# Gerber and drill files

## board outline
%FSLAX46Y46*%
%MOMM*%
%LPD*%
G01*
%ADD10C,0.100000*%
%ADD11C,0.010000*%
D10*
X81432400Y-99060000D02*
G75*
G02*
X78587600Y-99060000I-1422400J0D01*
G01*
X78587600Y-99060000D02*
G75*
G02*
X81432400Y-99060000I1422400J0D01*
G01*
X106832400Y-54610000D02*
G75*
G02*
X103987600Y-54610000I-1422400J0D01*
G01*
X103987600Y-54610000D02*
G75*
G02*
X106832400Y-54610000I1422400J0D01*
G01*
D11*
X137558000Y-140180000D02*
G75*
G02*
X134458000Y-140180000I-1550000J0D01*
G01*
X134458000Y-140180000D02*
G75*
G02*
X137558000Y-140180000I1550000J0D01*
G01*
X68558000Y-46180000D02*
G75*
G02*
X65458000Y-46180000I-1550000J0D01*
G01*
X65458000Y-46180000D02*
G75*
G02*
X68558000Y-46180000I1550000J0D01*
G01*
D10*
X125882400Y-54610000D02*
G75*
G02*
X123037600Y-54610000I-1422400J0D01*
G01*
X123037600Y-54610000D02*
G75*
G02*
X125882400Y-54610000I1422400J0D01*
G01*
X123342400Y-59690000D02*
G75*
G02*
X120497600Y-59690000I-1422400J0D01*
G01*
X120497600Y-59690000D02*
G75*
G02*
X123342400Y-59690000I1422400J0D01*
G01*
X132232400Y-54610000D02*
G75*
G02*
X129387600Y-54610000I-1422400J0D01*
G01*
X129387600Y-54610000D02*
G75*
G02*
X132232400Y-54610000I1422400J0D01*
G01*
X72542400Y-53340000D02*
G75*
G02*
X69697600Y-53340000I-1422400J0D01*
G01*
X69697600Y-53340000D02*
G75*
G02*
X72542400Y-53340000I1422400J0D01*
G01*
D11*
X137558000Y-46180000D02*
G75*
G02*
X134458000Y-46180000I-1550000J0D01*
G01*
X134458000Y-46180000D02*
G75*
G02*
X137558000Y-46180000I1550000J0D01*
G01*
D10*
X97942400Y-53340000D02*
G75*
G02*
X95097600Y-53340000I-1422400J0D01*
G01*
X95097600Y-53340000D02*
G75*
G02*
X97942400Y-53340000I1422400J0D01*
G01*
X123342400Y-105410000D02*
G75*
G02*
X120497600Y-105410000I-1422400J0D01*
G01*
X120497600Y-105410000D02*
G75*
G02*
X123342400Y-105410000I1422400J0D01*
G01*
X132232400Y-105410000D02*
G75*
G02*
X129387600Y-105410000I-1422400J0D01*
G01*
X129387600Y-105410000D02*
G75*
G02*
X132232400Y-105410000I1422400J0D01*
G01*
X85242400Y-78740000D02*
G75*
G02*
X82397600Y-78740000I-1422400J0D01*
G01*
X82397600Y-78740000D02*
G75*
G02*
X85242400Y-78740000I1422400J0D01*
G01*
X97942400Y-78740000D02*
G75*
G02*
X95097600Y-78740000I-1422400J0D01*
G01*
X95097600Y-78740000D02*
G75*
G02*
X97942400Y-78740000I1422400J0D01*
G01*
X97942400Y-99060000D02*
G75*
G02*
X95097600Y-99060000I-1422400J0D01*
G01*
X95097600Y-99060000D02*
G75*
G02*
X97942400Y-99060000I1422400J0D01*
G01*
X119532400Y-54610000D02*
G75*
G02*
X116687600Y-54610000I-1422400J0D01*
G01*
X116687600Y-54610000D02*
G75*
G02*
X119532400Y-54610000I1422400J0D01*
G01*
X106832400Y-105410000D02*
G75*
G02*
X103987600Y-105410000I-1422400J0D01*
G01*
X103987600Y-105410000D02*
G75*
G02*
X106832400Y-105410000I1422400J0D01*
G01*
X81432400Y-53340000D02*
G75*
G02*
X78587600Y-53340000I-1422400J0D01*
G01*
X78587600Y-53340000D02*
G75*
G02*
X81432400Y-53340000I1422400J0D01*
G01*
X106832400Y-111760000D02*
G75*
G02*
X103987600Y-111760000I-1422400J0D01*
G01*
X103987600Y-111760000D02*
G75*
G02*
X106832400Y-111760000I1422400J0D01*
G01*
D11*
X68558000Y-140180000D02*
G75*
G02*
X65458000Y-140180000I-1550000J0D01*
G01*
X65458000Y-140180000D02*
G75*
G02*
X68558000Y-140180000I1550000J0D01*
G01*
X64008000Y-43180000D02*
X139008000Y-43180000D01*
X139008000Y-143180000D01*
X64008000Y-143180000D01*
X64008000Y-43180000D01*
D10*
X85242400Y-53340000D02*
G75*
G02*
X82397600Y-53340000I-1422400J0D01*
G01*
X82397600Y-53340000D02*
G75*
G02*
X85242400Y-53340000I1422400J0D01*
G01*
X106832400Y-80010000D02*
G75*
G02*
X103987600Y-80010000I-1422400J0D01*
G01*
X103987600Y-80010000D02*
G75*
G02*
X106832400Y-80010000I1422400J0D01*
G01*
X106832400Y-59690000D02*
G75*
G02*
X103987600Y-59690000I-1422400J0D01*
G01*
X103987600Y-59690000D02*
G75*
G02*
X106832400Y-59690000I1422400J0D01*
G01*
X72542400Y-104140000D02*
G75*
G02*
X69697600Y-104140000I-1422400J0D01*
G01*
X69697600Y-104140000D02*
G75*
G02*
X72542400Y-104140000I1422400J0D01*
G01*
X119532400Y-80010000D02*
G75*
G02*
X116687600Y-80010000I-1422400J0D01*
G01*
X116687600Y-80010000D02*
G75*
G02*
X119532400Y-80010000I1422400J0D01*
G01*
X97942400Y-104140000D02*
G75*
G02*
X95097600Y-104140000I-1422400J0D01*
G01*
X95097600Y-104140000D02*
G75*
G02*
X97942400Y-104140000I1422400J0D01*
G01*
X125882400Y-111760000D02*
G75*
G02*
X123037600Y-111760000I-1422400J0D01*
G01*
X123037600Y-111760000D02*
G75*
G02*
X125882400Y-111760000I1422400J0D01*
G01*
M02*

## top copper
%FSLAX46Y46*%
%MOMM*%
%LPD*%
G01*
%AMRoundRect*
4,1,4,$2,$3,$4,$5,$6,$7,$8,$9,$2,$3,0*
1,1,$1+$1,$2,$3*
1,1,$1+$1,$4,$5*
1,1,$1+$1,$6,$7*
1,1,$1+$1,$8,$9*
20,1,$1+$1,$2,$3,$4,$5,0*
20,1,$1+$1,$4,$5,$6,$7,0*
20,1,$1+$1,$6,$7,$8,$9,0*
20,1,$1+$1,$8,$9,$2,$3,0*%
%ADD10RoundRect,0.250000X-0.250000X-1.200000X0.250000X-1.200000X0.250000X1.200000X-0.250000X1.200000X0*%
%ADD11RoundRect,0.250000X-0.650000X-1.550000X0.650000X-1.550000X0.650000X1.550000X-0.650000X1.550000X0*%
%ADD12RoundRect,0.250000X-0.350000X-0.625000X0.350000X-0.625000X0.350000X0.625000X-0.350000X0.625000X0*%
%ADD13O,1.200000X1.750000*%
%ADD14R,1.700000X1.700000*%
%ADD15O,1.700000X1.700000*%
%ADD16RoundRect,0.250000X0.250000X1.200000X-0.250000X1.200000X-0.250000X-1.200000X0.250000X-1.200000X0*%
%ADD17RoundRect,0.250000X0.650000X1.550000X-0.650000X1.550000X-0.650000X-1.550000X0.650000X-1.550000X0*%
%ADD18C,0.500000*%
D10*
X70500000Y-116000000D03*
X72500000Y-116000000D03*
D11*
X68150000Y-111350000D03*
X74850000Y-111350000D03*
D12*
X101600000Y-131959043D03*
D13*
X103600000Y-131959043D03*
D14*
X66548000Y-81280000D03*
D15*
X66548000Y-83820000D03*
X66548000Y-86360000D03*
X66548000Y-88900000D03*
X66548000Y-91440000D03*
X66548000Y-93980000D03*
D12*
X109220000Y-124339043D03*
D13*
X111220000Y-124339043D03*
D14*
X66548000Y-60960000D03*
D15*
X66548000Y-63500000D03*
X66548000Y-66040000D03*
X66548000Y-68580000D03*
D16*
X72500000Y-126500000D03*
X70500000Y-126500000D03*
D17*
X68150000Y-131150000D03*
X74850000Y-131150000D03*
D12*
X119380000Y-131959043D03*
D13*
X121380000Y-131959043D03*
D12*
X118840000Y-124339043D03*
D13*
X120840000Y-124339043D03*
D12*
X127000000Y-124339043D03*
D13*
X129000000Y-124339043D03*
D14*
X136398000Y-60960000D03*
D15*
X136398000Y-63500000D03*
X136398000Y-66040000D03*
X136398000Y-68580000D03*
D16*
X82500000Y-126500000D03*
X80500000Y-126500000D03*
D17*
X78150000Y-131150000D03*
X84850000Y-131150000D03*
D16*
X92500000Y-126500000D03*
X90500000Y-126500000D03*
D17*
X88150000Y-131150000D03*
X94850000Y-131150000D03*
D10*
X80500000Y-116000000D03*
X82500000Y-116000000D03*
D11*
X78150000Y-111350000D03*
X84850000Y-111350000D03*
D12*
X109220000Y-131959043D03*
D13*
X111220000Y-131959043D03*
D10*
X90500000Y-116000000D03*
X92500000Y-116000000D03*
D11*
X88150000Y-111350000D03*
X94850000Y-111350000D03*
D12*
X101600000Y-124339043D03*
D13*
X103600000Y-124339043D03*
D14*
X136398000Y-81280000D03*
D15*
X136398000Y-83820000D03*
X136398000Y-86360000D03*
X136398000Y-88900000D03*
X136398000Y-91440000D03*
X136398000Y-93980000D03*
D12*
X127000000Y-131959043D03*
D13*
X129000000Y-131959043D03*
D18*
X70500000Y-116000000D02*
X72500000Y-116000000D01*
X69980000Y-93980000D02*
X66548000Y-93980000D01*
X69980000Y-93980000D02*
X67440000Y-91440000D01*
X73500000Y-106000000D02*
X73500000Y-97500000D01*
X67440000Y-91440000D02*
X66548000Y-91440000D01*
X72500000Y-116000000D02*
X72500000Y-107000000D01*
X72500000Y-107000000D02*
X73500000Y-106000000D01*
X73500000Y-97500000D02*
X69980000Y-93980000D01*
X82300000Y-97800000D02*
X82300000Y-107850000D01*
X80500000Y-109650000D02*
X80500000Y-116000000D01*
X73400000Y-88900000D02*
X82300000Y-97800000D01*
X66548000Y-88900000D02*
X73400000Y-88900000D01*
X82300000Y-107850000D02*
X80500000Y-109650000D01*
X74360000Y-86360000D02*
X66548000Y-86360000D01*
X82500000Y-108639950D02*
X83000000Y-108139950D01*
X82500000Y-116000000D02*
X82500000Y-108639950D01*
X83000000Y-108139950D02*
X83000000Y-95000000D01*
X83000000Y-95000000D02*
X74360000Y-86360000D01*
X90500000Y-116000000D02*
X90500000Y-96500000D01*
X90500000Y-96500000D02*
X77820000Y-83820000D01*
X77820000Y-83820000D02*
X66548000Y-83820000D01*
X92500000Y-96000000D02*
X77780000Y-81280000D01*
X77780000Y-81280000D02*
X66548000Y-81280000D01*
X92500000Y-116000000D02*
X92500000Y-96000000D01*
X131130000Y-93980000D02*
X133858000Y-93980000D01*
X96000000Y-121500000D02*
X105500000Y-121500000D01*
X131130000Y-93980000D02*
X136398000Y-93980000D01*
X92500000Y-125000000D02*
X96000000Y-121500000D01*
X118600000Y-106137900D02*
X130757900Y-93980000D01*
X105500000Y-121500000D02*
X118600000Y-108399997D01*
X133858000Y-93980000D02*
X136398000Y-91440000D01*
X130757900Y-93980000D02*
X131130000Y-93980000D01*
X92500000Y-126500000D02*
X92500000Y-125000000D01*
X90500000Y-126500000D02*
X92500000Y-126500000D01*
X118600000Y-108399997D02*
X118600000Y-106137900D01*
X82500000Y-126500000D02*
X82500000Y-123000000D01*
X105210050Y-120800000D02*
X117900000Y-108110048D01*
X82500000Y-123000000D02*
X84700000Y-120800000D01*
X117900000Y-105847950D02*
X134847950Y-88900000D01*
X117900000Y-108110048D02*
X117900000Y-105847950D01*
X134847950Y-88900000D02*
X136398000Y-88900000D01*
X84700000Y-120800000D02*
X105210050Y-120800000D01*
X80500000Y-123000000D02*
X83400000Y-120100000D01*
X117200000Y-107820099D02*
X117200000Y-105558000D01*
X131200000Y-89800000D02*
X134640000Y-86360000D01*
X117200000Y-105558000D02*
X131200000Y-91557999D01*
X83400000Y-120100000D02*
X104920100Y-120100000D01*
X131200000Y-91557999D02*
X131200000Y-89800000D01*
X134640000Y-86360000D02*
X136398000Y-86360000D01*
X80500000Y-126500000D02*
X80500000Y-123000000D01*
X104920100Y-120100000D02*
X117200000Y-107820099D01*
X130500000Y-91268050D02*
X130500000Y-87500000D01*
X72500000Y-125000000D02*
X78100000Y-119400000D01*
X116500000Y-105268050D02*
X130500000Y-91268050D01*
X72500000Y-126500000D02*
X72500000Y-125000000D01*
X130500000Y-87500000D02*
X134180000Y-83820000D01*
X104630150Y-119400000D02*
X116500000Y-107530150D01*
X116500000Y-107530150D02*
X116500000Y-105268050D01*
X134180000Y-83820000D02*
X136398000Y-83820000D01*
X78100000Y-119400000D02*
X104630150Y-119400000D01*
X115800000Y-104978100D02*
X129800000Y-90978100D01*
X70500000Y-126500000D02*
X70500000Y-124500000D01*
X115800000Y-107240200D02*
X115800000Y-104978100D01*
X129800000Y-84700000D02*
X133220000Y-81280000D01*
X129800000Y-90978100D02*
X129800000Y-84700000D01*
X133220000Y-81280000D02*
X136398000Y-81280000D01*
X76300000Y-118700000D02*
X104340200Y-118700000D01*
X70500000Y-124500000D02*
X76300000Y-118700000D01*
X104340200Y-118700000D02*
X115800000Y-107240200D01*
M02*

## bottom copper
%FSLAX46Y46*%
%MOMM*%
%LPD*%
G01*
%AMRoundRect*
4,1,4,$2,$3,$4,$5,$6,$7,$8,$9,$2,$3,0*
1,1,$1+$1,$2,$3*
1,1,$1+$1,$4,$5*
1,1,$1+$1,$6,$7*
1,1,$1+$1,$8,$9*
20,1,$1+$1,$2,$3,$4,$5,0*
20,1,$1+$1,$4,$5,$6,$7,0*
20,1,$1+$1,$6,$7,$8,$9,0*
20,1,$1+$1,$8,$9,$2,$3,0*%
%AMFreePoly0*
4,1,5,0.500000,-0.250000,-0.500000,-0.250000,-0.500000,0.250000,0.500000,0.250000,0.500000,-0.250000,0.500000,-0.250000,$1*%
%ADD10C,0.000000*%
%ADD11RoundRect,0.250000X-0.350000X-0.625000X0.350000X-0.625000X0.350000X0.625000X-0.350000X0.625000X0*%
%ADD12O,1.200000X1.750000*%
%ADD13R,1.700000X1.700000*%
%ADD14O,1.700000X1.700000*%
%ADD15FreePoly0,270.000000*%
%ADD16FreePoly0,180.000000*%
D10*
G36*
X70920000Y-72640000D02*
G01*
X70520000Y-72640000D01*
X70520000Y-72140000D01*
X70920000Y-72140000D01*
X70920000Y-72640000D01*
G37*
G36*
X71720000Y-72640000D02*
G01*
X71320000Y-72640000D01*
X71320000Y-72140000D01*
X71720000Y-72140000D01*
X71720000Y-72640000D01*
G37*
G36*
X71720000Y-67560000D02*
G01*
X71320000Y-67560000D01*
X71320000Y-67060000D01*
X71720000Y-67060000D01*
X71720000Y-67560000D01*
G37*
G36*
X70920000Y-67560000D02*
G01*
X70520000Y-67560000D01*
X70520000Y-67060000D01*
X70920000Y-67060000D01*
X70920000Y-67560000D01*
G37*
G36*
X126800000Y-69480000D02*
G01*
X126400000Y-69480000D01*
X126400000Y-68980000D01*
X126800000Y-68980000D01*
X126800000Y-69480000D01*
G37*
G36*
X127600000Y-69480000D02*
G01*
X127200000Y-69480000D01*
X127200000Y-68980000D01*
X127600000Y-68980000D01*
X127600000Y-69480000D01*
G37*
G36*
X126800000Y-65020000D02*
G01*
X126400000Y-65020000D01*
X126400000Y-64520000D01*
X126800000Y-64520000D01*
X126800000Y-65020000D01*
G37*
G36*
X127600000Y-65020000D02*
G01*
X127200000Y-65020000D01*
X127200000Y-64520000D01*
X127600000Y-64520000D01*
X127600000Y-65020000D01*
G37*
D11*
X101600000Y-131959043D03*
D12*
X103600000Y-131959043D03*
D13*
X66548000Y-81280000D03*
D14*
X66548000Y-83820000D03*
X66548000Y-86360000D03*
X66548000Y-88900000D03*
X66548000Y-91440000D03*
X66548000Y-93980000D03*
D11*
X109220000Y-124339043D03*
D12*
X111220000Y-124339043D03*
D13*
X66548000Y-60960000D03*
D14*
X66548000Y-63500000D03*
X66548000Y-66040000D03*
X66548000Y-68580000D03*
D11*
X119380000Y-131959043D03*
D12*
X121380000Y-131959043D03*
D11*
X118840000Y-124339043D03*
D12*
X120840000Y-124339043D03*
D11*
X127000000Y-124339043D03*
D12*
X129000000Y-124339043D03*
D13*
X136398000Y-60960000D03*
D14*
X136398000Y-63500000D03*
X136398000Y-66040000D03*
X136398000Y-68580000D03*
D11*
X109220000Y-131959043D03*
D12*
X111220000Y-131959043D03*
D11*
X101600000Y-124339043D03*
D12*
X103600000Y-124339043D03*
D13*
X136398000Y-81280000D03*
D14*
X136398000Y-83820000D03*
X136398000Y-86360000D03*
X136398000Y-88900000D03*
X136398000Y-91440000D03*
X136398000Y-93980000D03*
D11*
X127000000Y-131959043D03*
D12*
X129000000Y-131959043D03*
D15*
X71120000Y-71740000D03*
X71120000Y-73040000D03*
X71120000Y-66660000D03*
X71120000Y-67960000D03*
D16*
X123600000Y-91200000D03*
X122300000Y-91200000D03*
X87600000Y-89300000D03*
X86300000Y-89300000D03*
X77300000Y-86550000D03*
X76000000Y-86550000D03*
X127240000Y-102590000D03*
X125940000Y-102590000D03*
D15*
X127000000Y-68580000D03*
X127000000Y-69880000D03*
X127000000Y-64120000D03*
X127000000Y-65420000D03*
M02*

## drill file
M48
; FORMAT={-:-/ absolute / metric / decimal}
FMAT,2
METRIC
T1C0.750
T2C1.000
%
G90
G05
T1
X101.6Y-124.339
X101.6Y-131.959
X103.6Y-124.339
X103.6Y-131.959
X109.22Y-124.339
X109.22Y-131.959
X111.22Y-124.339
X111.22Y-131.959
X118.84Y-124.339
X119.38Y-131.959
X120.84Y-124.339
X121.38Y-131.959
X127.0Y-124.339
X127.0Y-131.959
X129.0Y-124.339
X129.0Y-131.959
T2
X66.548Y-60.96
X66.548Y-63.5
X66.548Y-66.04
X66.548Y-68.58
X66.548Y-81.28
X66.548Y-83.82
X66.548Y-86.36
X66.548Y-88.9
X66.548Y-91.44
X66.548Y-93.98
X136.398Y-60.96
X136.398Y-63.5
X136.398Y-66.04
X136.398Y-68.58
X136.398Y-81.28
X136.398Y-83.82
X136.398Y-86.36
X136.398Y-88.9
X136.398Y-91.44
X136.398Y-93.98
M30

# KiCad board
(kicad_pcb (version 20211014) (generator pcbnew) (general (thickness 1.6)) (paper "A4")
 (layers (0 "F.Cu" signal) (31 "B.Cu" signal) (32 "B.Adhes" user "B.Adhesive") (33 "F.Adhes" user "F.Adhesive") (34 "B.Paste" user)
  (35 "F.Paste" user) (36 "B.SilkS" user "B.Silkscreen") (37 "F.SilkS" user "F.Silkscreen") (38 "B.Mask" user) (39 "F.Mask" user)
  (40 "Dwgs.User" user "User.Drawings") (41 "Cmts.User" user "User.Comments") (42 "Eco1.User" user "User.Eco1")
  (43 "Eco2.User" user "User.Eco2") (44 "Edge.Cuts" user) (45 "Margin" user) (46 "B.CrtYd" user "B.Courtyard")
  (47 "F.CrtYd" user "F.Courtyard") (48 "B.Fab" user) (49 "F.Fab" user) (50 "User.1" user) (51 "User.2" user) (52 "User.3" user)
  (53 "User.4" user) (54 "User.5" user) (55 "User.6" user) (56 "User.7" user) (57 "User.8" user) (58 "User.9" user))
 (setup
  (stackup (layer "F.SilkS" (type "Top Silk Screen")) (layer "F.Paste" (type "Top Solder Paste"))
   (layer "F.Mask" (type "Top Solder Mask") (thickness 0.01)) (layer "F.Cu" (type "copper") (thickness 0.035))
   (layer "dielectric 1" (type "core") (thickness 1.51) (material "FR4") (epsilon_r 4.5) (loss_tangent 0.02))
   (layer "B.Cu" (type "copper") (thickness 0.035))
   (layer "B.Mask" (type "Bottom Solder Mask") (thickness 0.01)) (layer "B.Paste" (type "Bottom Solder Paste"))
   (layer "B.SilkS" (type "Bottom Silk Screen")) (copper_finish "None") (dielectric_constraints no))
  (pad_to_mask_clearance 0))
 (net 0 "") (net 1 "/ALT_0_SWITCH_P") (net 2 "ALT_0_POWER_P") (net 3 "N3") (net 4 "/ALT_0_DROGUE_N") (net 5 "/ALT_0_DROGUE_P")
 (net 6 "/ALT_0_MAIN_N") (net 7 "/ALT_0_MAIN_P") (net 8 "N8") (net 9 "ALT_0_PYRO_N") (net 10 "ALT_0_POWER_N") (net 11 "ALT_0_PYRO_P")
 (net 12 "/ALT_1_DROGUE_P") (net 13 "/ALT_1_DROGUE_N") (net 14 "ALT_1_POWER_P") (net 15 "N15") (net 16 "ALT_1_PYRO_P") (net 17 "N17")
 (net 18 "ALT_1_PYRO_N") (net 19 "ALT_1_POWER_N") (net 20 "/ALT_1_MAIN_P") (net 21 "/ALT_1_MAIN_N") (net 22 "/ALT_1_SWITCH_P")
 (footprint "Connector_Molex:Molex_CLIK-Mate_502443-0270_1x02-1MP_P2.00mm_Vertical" (layer "F.Cu") (at 71.5 113.5)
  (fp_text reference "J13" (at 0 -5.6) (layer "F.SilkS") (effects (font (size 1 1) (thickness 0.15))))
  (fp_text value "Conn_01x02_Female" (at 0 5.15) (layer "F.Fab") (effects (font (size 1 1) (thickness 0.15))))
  (pad "1" smd roundrect (at -1 2.5) (size 1 2.9) (layers "F.Cu" "F.Paste" "F.Mask") (roundrect_rratio 0.25) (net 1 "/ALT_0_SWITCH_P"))
  (pad "2" smd roundrect (at 1 2.5) (size 1 2.9) (layers "F.Cu" "F.Paste" "F.Mask") (roundrect_rratio 0.25) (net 1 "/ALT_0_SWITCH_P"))
  (pad "MP" smd roundrect (at -3.35 -2.15) (size 1.8 3.6) (layers "F.Cu" "F.Paste" "F.Mask") (roundrect_rratio 0.138889))
  (pad "MP" smd roundrect (at 3.35 -2.15) (size 1.8 3.6) (layers "F.Cu" "F.Paste" "F.Mask") (roundrect_rratio 0.138889)))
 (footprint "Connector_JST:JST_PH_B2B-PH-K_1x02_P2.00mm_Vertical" (layer "F.Cu") (at 101.6 131.959043)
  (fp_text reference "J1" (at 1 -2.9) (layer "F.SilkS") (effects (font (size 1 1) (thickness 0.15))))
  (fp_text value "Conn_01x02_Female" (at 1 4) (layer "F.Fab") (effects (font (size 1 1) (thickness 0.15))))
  (pad "1" thru_hole roundrect (at 0 0) (size 1.2 1.75) (drill 0.75) (layers *.Cu *.Mask) (roundrect_rratio 0.208333)
   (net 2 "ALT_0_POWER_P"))
  (pad "2" thru_hole oval (at 2 0) (size 1.2 1.75) (drill 0.75) (layers *.Cu *.Mask) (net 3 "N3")))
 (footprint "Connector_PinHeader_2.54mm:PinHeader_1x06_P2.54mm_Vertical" (layer "F.Cu") (at 66.548 81.28)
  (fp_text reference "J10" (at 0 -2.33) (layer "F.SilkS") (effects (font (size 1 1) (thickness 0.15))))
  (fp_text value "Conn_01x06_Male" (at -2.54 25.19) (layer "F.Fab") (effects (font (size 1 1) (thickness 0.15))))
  (pad "1" thru_hole rect (at 0 0) (size 1.7 1.7) (drill 1) (layers *.Cu *.Mask) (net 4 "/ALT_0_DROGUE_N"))
  (pad "2" thru_hole oval (at 0 2.54) (size 1.7 1.7) (drill 1) (layers *.Cu *.Mask) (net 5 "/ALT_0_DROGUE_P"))
  (pad "3" thru_hole oval (at 0 5.08) (size 1.7 1.7) (drill 1) (layers *.Cu *.Mask) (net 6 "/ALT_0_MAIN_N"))
  (pad "4" thru_hole oval (at 0 7.62) (size 1.7 1.7) (drill 1) (layers *.Cu *.Mask) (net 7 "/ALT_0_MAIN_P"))
  (pad "5" thru_hole oval (at 0 10.16) (size 1.7 1.7) (drill 1) (layers *.Cu *.Mask) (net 1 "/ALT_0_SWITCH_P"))
  (pad "6" thru_hole oval (at 0 12.7) (size 1.7 1.7) (drill 1) (layers *.Cu *.Mask) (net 1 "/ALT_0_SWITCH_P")))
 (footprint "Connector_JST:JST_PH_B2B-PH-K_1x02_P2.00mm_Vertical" (layer "F.Cu") (at 109.22 124.339043)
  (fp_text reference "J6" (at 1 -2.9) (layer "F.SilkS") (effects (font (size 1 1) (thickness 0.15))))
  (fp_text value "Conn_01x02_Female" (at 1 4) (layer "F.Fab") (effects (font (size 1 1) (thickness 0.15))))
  (pad "1" thru_hole roundrect (at 0 0) (size 1.2 1.75) (drill 0.75) (layers *.Cu *.Mask) (roundrect_rratio 0.208333) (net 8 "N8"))
  (pad "2" thru_hole oval (at 2 0) (size 1.2 1.75) (drill 0.75) (layers *.Cu *.Mask) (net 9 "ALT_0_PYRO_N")))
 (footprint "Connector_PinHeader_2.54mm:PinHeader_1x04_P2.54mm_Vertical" (layer "F.Cu") (at 66.548 60.96)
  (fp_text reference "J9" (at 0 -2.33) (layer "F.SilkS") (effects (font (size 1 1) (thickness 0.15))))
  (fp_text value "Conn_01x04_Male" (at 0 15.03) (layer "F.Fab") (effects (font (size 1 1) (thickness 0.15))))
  (pad "1" thru_hole rect (at 0 0) (size 1.7 1.7) (drill 1) (layers *.Cu *.Mask) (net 2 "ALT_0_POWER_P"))
  (pad "2" thru_hole oval (at 0 2.54) (size 1.7 1.7) (drill 1) (layers *.Cu *.Mask) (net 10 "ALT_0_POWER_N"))
  (pad "3" thru_hole oval (at 0 5.08) (size 1.7 1.7) (drill 1) (layers *.Cu *.Mask) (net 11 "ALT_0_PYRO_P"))
  (pad "4" thru_hole oval (at 0 7.62) (size 1.7 1.7) (drill 1) (layers *.Cu *.Mask) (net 9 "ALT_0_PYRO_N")))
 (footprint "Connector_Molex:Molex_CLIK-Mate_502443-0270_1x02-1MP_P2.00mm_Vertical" (layer "F.Cu") (at 71.5 129 180)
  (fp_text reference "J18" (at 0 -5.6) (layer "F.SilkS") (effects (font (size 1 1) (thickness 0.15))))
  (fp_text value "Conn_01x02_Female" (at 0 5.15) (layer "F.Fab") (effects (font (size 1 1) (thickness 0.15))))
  (pad "1" smd roundrect (at -1 2.5 180) (size 1 2.9) (layers "F.Cu" "F.Paste" "F.Mask") (roundrect_rratio 0.25) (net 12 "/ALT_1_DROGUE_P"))
  (pad "2" smd roundrect (at 1 2.5 180) (size 1 2.9) (layers "F.Cu" "F.Paste" "F.Mask") (roundrect_rratio 0.25) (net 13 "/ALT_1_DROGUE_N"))
  (pad "MP" smd roundrect (at 3.35 -2.15 180) (size 1.8 3.6) (layers "F.Cu" "F.Paste" "F.Mask") (roundrect_rratio 0.138889))
  (pad "MP" smd roundrect (at -3.35 -2.15 180) (size 1.8 3.6) (layers "F.Cu" "F.Paste" "F.Mask") (roundrect_rratio 0.138889)))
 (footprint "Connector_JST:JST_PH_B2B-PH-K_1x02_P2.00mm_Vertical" (layer "F.Cu") (at 119.38 131.959043)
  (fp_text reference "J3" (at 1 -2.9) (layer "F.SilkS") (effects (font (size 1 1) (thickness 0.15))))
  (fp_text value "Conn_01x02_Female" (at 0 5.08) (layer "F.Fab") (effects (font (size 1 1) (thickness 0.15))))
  (pad "1" thru_hole roundrect (at 0 0) (size 1.2 1.75) (drill 0.75) (layers *.Cu *.Mask) (roundrect_rratio 0.208333)
   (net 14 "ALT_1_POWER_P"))
  (pad "2" thru_hole oval (at 2 0) (size 1.2 1.75) (drill 0.75) (layers *.Cu *.Mask) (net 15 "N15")))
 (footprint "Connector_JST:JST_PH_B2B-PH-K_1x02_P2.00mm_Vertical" (layer "F.Cu") (at 118.84 124.339043)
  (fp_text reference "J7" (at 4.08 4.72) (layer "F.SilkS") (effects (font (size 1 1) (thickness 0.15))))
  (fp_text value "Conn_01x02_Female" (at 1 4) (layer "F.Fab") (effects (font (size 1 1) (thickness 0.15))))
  (pad "1" thru_hole roundrect (at 0 0) (size 1.2 1.75) (drill 0.75) (layers *.Cu *.Mask) (roundrect_rratio 0.208333)
   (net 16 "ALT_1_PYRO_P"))
  (pad "2" thru_hole oval (at 2 0) (size 1.2 1.75) (drill 0.75) (layers *.Cu *.Mask) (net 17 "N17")))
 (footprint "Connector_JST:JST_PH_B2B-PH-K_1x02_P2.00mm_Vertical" (layer "F.Cu") (at 127 124.339043)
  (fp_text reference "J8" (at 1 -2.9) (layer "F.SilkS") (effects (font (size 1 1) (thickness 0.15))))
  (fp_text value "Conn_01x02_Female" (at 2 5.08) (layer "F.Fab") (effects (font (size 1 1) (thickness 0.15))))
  (pad "1" thru_hole roundrect (at 0 0) (size 1.2 1.75) (drill 0.75) (layers *.Cu *.Mask) (roundrect_rratio 0.208333) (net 17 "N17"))
  (pad "2" thru_hole oval (at 2 0) (size 1.2 1.75) (drill 0.75) (layers *.Cu *.Mask) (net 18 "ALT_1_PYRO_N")))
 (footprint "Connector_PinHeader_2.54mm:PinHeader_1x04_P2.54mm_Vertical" (layer "F.Cu") (at 136.398 60.96)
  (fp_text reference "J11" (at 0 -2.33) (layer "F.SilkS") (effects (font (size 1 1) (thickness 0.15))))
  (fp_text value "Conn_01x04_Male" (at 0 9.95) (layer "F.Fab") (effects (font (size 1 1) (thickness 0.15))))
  (pad "1" thru_hole rect (at 0 0) (size 1.7 1.7) (drill 1) (layers *.Cu *.Mask) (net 14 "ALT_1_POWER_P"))
  (pad "2" thru_hole oval (at 0 2.54) (size 1.7 1.7) (drill 1) (layers *.Cu *.Mask) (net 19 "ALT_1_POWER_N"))
  (pad "3" thru_hole oval (at 0 5.08) (size 1.7 1.7) (drill 1) (layers *.Cu *.Mask) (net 16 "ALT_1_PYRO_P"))
  (pad "4" thru_hole oval (at 0 7.62) (size 1.7 1.7) (drill 1) (layers *.Cu *.Mask) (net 18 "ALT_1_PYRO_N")))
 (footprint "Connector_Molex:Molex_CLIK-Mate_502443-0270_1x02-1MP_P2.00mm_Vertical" (layer "F.Cu") (at 81.5 129 180)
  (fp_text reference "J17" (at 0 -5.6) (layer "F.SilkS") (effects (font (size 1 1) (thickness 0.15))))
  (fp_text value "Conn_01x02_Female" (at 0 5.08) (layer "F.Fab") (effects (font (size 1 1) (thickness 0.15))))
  (pad "1" smd roundrect (at -1 2.5 180) (size 1 2.9) (layers "F.Cu" "F.Paste" "F.Mask") (roundrect_rratio 0.25) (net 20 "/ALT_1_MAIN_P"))
  (pad "2" smd roundrect (at 1 2.5 180) (size 1 2.9) (layers "F.Cu" "F.Paste" "F.Mask") (roundrect_rratio 0.25) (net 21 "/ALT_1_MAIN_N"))
  (pad "MP" smd roundrect (at 3.35 -2.15 180) (size 1.8 3.6) (layers "F.Cu" "F.Paste" "F.Mask") (roundrect_rratio 0.138889))
  (pad "MP" smd roundrect (at -3.35 -2.15 180) (size 1.8 3.6) (layers "F.Cu" "F.Paste" "F.Mask") (roundrect_rratio 0.138889)))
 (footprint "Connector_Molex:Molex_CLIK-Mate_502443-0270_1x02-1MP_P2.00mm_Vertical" (layer "F.Cu") (at 91.5 129 180)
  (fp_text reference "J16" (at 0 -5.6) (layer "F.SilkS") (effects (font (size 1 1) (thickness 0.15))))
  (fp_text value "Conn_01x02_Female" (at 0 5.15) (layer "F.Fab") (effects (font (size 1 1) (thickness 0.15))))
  (pad "1" smd roundrect (at -1 2.5 180) (size 1 2.9) (layers "F.Cu" "F.Paste" "F.Mask") (roundrect_rratio 0.25) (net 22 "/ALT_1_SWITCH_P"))
  (pad "2" smd roundrect (at 1 2.5 180) (size 1 2.9) (layers "F.Cu" "F.Paste" "F.Mask") (roundrect_rratio 0.25) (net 22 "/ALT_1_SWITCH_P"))
  (pad "MP" smd roundrect (at 3.35 -2.15 180) (size 1.8 3.6) (layers "F.Cu" "F.Paste" "F.Mask") (roundrect_rratio 0.138889))
  (pad "MP" smd roundrect (at -3.35 -2.15 180) (size 1.8 3.6) (layers "F.Cu" "F.Paste" "F.Mask") (roundrect_rratio 0.138889)))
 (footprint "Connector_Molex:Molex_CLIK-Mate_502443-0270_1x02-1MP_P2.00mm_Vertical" (layer "F.Cu") (at 81.5 113.5)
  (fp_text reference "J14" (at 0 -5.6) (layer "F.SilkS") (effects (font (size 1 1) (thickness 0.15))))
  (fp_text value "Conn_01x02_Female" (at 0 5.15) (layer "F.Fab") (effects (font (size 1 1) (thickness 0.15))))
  (pad "1" smd roundrect (at -1 2.5) (size 1 2.9) (layers "F.Cu" "F.Paste" "F.Mask") (roundrect_rratio 0.25) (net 7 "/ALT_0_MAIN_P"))
  (pad "2" smd roundrect (at 1 2.5) (size 1 2.9) (layers "F.Cu" "F.Paste" "F.Mask") (roundrect_rratio 0.25) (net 6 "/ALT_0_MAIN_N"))
  (pad "MP" smd roundrect (at -3.35 -2.15) (size 1.8 3.6) (layers "F.Cu" "F.Paste" "F.Mask") (roundrect_rratio 0.138889))
  (pad "MP" smd roundrect (at 3.35 -2.15) (size 1.8 3.6) (layers "F.Cu" "F.Paste" "F.Mask") (roundrect_rratio 0.138889)))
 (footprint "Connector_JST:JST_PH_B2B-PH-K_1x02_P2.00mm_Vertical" (layer "F.Cu") (at 109.22 131.959043)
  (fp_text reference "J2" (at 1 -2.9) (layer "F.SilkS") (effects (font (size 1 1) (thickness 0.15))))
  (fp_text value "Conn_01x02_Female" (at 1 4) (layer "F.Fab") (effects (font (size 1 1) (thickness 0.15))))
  (pad "1" thru_hole roundrect (at 0 0) (size 1.2 1.75) (drill 0.75) (layers *.Cu *.Mask) (roundrect_rratio 0.208333) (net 3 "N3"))
  (pad "2" thru_hole oval (at 2 0) (size 1.2 1.75) (drill 0.75) (layers *.Cu *.Mask) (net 10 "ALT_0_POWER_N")))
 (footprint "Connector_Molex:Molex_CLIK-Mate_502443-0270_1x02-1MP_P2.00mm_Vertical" (layer "F.Cu") (at 91.5 113.5)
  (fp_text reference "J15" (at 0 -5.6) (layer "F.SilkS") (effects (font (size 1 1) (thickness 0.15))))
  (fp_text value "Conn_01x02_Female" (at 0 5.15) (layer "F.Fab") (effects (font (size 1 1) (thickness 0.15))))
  (pad "1" smd roundrect (at -1 2.5) (size 1 2.9) (layers "F.Cu" "F.Paste" "F.Mask") (roundrect_rratio 0.25) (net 5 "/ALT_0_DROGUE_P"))
  (pad "2" smd roundrect (at 1 2.5) (size 1 2.9) (layers "F.Cu" "F.Paste" "F.Mask") (roundrect_rratio 0.25) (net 4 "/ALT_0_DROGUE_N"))
  (pad "MP" smd roundrect (at -3.35 -2.15) (size 1.8 3.6) (layers "F.Cu" "F.Paste" "F.Mask") (roundrect_rratio 0.138889))
  (pad "MP" smd roundrect (at 3.35 -2.15) (size 1.8 3.6) (layers "F.Cu" "F.Paste" "F.Mask") (roundrect_rratio 0.138889)))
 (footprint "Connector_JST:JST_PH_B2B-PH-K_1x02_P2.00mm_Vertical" (layer "F.Cu") (at 101.6 124.339043)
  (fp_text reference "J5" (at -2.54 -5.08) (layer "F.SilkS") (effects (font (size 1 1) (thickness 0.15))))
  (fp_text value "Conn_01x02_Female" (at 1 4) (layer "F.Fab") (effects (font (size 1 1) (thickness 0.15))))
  (pad "1" thru_hole roundrect (at 0 0) (size 1.2 1.75) (drill 0.75) (layers *.Cu *.Mask) (roundrect_rratio 0.208333)
   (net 11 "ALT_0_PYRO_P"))
  (pad "2" thru_hole oval (at 2 0) (size 1.2 1.75) (drill 0.75) (layers *.Cu *.Mask) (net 8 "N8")))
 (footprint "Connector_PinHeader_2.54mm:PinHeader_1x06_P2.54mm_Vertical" (layer "F.Cu") (at 136.398 81.28)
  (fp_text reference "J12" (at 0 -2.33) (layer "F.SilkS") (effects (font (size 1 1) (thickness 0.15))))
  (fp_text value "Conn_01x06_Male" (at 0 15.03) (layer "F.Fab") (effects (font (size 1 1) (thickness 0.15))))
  (pad "1" thru_hole rect (at 0 0) (size 1.7 1.7) (drill 1) (layers *.Cu *.Mask) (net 13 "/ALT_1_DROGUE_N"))
  (pad "2" thru_hole oval (at 0 2.54) (size 1.7 1.7) (drill 1) (layers *.Cu *.Mask) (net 12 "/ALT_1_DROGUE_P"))
  (pad "3" thru_hole oval (at 0 5.08) (size 1.7 1.7) (drill 1) (layers *.Cu *.Mask) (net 21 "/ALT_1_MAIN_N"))
  (pad "4" thru_hole oval (at 0 7.62) (size 1.7 1.7) (drill 1) (layers *.Cu *.Mask) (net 20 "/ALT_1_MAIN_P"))
  (pad "5" thru_hole oval (at 0 10.16) (size 1.7 1.7) (drill 1) (layers *.Cu *.Mask) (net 22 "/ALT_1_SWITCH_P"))
  (pad "6" thru_hole oval (at 0 12.7) (size 1.7 1.7) (drill 1) (layers *.Cu *.Mask) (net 22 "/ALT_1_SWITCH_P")))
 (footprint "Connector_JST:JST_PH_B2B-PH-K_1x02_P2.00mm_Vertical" (layer "F.Cu") (at 127 131.959043)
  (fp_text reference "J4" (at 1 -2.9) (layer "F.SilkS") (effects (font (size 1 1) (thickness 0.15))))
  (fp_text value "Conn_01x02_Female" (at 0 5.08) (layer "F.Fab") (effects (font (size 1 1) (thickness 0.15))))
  (pad "1" thru_hole roundrect (at 0 0) (size 1.2 1.75) (drill 0.75) (layers *.Cu *.Mask) (roundrect_rratio 0.208333) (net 15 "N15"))
  (pad "2" thru_hole oval (at 2 0) (size 1.2 1.75) (drill 0.75) (layers *.Cu *.Mask) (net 19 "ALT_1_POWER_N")))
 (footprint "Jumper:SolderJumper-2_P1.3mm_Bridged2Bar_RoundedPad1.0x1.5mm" (layer "B.Cu") (at 71.12 72.39 -90)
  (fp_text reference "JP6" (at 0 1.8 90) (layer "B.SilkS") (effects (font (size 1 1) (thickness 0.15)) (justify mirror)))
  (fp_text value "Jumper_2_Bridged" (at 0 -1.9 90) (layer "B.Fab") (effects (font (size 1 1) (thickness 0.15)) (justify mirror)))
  (fp_poly (pts (xy -0.25 0.6) (xy 0.25 0.6) (xy 0.25 0.2) (xy -0.25 0.2)) (layer "B.Cu") (width 0) (fill solid))
  (fp_poly (pts (xy -0.25 -0.2) (xy 0.25 -0.2) (xy 0.25 -0.6) (xy -0.25 -0.6)) (layer "B.Cu") (width 0) (fill solid))
  (pad "1" smd custom (at -0.65 0 270) (size 1 0.5) (layers "B.Cu" "B.Mask") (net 10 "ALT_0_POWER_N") (zone_connect 2)
   (options (clearance outline) (anchor rect)) (primitives))
  (pad "2" smd custom (at 0.65 0 270) (size 1 0.5) (layers "B.Cu" "B.Mask") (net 9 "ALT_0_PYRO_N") (zone_connect 2)
   (options (clearance outline) (anchor rect)) (primitives)))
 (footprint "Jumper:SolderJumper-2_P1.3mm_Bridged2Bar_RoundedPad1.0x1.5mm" (layer "B.Cu") (at 71.12 67.31 -90)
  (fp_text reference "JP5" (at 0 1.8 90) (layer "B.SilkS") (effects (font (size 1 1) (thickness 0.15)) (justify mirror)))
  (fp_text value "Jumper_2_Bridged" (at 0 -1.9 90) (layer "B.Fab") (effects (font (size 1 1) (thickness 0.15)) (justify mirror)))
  (fp_poly (pts (xy -0.25 -0.2) (xy 0.25 -0.2) (xy 0.25 -0.6) (xy -0.25 -0.6)) (layer "B.Cu") (width 0) (fill solid))
  (fp_poly (pts (xy -0.25 0.6) (xy 0.25 0.6) (xy 0.25 0.2) (xy -0.25 0.2)) (layer "B.Cu") (width 0) (fill solid))
  (pad "1" smd custom (at -0.65 0 270) (size 1 0.5) (layers "B.Cu" "B.Mask") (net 2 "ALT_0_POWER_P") (zone_connect 2)
   (options (clearance outline) (anchor rect)) (primitives))
  (pad "2" smd custom (at 0.65 0 270) (size 1 0.5) (layers "B.Cu" "B.Mask") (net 11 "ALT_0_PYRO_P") (zone_connect 2)
   (options (clearance outline) (anchor rect)) (primitives)))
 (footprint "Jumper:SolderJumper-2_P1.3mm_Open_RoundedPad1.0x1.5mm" (layer "B.Cu") (at 122.95 91.2 180)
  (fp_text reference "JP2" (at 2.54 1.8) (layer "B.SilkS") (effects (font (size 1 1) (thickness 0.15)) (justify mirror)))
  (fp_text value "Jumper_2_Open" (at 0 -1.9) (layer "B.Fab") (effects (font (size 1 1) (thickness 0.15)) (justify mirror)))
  (pad "1" smd custom (at -0.65 0 180) (size 1 0.5) (layers "B.Cu" "B.Mask") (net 19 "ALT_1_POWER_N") (zone_connect 2)
   (options (clearance outline) (anchor rect)) (primitives))
  (pad "2" smd custom (at 0.65 0 180) (size 1 0.5) (layers "B.Cu" "B.Mask") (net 15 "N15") (zone_connect 2)
   (options (clearance outline) (anchor rect)) (primitives)))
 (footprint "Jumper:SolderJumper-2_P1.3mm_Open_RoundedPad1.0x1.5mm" (layer "B.Cu") (at 86.95 89.3 180)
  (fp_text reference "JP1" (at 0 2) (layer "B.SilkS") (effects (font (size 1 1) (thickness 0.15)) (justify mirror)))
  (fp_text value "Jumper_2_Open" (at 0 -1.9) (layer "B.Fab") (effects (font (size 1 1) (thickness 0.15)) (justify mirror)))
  (pad "1" smd custom (at -0.65 0 180) (size 1 0.5) (layers "B.Cu" "B.Mask") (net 10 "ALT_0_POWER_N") (zone_connect 2)
   (options (clearance outline) (anchor rect)) (primitives))
  (pad "2" smd custom (at 0.65 0 180) (size 1 0.5) (layers "B.Cu" "B.Mask") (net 3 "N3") (zone_connect 2)
   (options (clearance outline) (anchor rect)) (primitives)))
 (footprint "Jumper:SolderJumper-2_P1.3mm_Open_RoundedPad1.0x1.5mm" (layer "B.Cu") (at 76.65 86.55 180)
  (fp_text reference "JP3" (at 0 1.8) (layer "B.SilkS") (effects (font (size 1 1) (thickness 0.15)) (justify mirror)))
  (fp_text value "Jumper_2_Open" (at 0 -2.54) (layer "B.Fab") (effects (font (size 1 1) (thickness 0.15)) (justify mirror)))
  (pad "1" smd custom (at -0.65 0 180) (size 1 0.5) (layers "B.Cu" "B.Mask") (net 9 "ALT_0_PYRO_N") (zone_connect 2)
   (options (clearance outline) (anchor rect)) (primitives))
  (pad "2" smd custom (at 0.65 0 180) (size 1 0.5) (layers "B.Cu" "B.Mask") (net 8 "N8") (zone_connect 2)
   (options (clearance outline) (anchor rect)) (primitives)))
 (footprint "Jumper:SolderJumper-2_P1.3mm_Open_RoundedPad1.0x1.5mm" (layer "B.Cu") (at 126.59 102.59 180)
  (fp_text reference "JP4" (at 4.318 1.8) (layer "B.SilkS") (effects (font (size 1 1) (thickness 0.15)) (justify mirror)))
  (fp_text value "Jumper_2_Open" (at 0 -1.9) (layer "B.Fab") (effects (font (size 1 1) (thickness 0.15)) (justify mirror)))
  (pad "1" smd custom (at -0.65 0 180) (size 1 0.5) (layers "B.Cu" "B.Mask") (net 18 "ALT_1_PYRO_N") (zone_connect 2)
   (options (clearance outline) (anchor rect)) (primitives))
  (pad "2" smd custom (at 0.65 0 180) (size 1 0.5) (layers "B.Cu" "B.Mask") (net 17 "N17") (zone_connect 2)
   (options (clearance outline) (anchor rect)) (primitives)))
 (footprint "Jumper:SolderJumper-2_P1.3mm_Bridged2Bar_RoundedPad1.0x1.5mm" (layer "B.Cu") (at 127 69.23 -90)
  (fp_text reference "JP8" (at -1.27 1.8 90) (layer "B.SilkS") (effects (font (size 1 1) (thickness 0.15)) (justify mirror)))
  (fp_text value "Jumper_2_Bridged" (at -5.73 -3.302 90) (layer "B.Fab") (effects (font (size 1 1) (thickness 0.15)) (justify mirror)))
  (fp_poly (pts (xy -0.25 0.6) (xy 0.25 0.6) (xy 0.25 0.2) (xy -0.25 0.2)) (layer "B.Cu") (width 0) (fill solid))
  (fp_poly (pts (xy -0.25 -0.2) (xy 0.25 -0.2) (xy 0.25 -0.6) (xy -0.25 -0.6)) (layer "B.Cu") (width 0) (fill solid))
  (pad "1" smd custom (at -0.65 0 270) (size 1 0.5) (layers "B.Cu" "B.Mask") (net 19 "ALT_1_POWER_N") (zone_connect 2)
   (options (clearance outline) (anchor rect)) (primitives))
  (pad "2" smd custom (at 0.65 0 270) (size 1 0.5) (layers "B.Cu" "B.Mask") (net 18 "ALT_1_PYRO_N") (zone_connect 2)
   (options (clearance outline) (anchor rect)) (primitives)))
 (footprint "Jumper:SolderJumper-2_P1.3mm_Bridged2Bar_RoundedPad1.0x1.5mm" (layer "B.Cu") (at 127 64.77 -90)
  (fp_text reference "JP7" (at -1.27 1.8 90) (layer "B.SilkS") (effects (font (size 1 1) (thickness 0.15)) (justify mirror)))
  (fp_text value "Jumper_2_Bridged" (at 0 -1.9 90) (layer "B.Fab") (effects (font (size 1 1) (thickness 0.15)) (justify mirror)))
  (fp_poly (pts (xy -0.25 0.6) (xy 0.25 0.6) (xy 0.25 0.2) (xy -0.25 0.2)) (layer "B.Cu") (width 0) (fill solid))
  (fp_poly (pts (xy -0.25 -0.2) (xy 0.25 -0.2) (xy 0.25 -0.6) (xy -0.25 -0.6)) (layer "B.Cu") (width 0) (fill solid))
  (pad "1" smd custom (at -0.65 0 270) (size 1 0.5) (layers "B.Cu" "B.Mask") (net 14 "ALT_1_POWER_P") (zone_connect 2)
   (options (clearance outline) (anchor rect)) (primitives))
  (pad "2" smd custom (at 0.65 0 270) (size 1 0.5) (layers "B.Cu" "B.Mask") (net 16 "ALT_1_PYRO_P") (zone_connect 2)
   (options (clearance outline) (anchor rect)) (primitives)))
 (gr_circle (center 80.01 99.06) (end 81.4324 99.06) (layer "Edge.Cuts") (width 0.1) (fill none))
 (gr_circle (center 105.41 54.61) (end 106.8324 54.61) (layer "Edge.Cuts") (width 0.1) (fill none))
 (gr_circle (center 136.008 140.18) (end 137.558 140.18) (layer "Edge.Cuts") (width 0.01) (fill none))
 (gr_circle (center 67.008 46.18) (end 68.558 46.18) (layer "Edge.Cuts") (width 0.01) (fill none))
 (gr_circle (center 124.46 54.61) (end 125.8824 54.61) (layer "Edge.Cuts") (width 0.1) (fill none))
 (gr_circle (center 121.92 59.69) (end 123.3424 59.69) (layer "Edge.Cuts") (width 0.1) (fill none))
 (gr_circle (center 130.81 54.61) (end 132.2324 54.61) (layer "Edge.Cuts") (width 0.1) (fill none))
 (gr_circle (center 71.12 53.34) (end 72.5424 53.34) (layer "Edge.Cuts") (width 0.1) (fill none))
 (gr_circle (center 136.008 46.18) (end 137.558 46.18) (layer "Edge.Cuts") (width 0.01) (fill none))
 (gr_circle (center 96.52 53.34) (end 97.9424 53.34) (layer "Edge.Cuts") (width 0.1) (fill none))
 (gr_circle (center 121.92 105.41) (end 123.3424 105.41) (layer "Edge.Cuts") (width 0.1) (fill none))
 (gr_circle (center 130.81 105.41) (end 132.2324 105.41) (layer "Edge.Cuts") (width 0.1) (fill none))
 (gr_circle (center 83.82 78.74) (end 85.2424 78.74) (layer "Edge.Cuts") (width 0.1) (fill none))
 (gr_circle (center 96.52 78.74) (end 97.9424 78.74) (layer "Edge.Cuts") (width 0.1) (fill none))
 (gr_circle (center 96.52 99.06) (end 97.9424 99.06) (layer "Edge.Cuts") (width 0.1) (fill none))
 (gr_circle (center 118.11 54.61) (end 119.5324 54.61) (layer "Edge.Cuts") (width 0.1) (fill none))
 (gr_circle (center 105.41 105.41) (end 106.8324 105.41) (layer "Edge.Cuts") (width 0.1) (fill none))
 (gr_circle (center 80.01 53.34) (end 81.4324 53.34) (layer "Edge.Cuts") (width 0.1) (fill none))
 (gr_circle (center 105.41 111.76) (end 106.8324 111.76) (layer "Edge.Cuts") (width 0.1) (fill none))
 (gr_circle (center 67.008 140.18) (end 68.558 140.18) (layer "Edge.Cuts") (width 0.01) (fill none))
 (gr_rect (start 64.008 43.18) (end 139.008 143.18) (layer "Edge.Cuts") (width 0.01) (fill none))
 (gr_circle (center 83.82 53.34) (end 85.2424 53.34) (layer "Edge.Cuts") (width 0.1) (fill none))
 (gr_circle (center 105.41 80.01) (end 106.8324 80.01) (layer "Edge.Cuts") (width 0.1) (fill none))
 (gr_circle (center 105.41 59.69) (end 106.8324 59.69) (layer "Edge.Cuts") (width 0.1) (fill none))
 (gr_circle (center 71.12 104.14) (end 72.5424 104.14) (layer "Edge.Cuts") (width 0.1) (fill none))
 (gr_circle (center 118.11 80.01) (end 119.5324 80.01) (layer "Edge.Cuts") (width 0.1) (fill none))
 (gr_circle (center 96.52 104.14) (end 97.9424 104.14) (layer "Edge.Cuts") (width 0.1) (fill none))
 (gr_circle (center 124.46 111.76) (end 125.8824 111.76) (layer "Edge.Cuts") (width 0.1) (fill none))
 (segment (start 70.5 116) (end 72.5 116) (width 0.5) (layer "F.Cu") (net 1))
 (segment (start 69.98 93.98) (end 66.548 93.98) (width 0.5) (layer "F.Cu") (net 1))
 (segment (start 69.98 93.98) (end 67.44 91.44) (width 0.5) (layer "F.Cu") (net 1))
 (segment (start 73.5 106) (end 73.5 97.5) (width 0.5) (layer "F.Cu") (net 1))
 (segment (start 67.44 91.44) (end 66.548 91.44) (width 0.5) (layer "F.Cu") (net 1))
 (segment (start 72.5 116) (end 72.5 107) (width 0.5) (layer "F.Cu") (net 1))
 (segment (start 72.5 107) (end 73.5 106) (width 0.5) (layer "F.Cu") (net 1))
 (segment (start 73.5 97.5) (end 69.98 93.98) (width 0.5) (layer "F.Cu") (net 1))
 (segment (start 82.3 97.8) (end 82.3 107.85) (width 0.5) (layer "F.Cu") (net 7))
 (segment (start 80.5 109.65) (end 80.5 116) (width 0.5) (layer "F.Cu") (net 7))
 (segment (start 73.4 88.9) (end 82.3 97.8) (width 0.5) (layer "F.Cu") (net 7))
 (segment (start 66.548 88.9) (end 73.4 88.9) (width 0.5) (layer "F.Cu") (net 7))
 (segment (start 82.3 107.85) (end 80.5 109.65) (width 0.5) (layer "F.Cu") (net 7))
 (segment (start 74.36 86.36) (end 66.548 86.36) (width 0.5) (layer "F.Cu") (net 6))
 (segment (start 82.5 108.63995) (end 83 108.13995) (width 0.5) (layer "F.Cu") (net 6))
 (segment (start 82.5 116) (end 82.5 108.63995) (width 0.5) (layer "F.Cu") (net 6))
 (segment (start 83 108.13995) (end 83 95) (width 0.5) (layer "F.Cu") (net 6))
 (segment (start 83 95) (end 74.36 86.36) (width 0.5) (layer "F.Cu") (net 6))
 (segment (start 90.5 116) (end 90.5 96.5) (width 0.5) (layer "F.Cu") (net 5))
 (segment (start 90.5 96.5) (end 77.82 83.82) (width 0.5) (layer "F.Cu") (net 5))
 (segment (start 77.82 83.82) (end 66.548 83.82) (width 0.5) (layer "F.Cu") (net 5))
 (segment (start 92.5 96) (end 77.78 81.28) (width 0.5) (layer "F.Cu") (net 4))
 (segment (start 77.78 81.28) (end 66.548 81.28) (width 0.5) (layer "F.Cu") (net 4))
 (segment (start 92.5 116) (end 92.5 96) (width 0.5) (layer "F.Cu") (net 4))
 (segment (start 131.13 93.98) (end 133.858 93.98) (width 0.5) (layer "F.Cu") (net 22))
 (segment (start 96 121.5) (end 105.5 121.5) (width 0.5) (layer "F.Cu") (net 22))
 (segment (start 131.13 93.98) (end 136.398 93.98) (width 0.5) (layer "F.Cu") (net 22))
 (segment (start 92.5 125) (end 96 121.5) (width 0.5) (layer "F.Cu") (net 22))
 (segment (start 118.6 106.1379) (end 130.7579 93.98) (width 0.5) (layer "F.Cu") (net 22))
 (segment (start 105.5 121.5) (end 118.6 108.399997) (width 0.5) (layer "F.Cu") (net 22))
 (segment (start 133.858 93.98) (end 136.398 91.44) (width 0.5) (layer "F.Cu") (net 22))
 (segment (start 130.7579 93.98) (end 131.13 93.98) (width 0.5) (layer "F.Cu") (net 22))
 (segment (start 92.5 126.5) (end 92.5 125) (width 0.5) (layer "F.Cu") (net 22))
 (segment (start 90.5 126.5) (end 92.5 126.5) (width 0.5) (layer "F.Cu") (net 22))
 (segment (start 118.6 108.399997) (end 118.6 106.1379) (width 0.5) (layer "F.Cu") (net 22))
 (segment (start 82.5 126.5) (end 82.5 123) (width 0.5) (layer "F.Cu") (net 20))
 (segment (start 105.21005 120.8) (end 117.9 108.110048) (width 0.5) (layer "F.Cu") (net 20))
 (segment (start 82.5 123) (end 84.7 120.8) (width 0.5) (layer "F.Cu") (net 20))
 (segment (start 117.9 105.84795) (end 134.84795 88.9) (width 0.5) (layer "F.Cu") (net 20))
 (segment (start 117.9 108.110048) (end 117.9 105.84795) (width 0.5) (layer "F.Cu") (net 20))
 (segment (start 134.84795 88.9) (end 136.398 88.9) (width 0.5) (layer "F.Cu") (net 20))
 (segment (start 84.7 120.8) (end 105.21005 120.8) (width 0.5) (layer "F.Cu") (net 20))
 (segment (start 80.5 123) (end 83.4 120.1) (width 0.5) (layer "F.Cu") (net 21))
 (segment (start 117.2 107.820099) (end 117.2 105.558) (width 0.5) (layer "F.Cu") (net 21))
 (segment (start 131.2 89.8) (end 134.64 86.36) (width 0.5) (layer "F.Cu") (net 21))
 (segment (start 117.2 105.558) (end 131.2 91.557999) (width 0.5) (layer "F.Cu") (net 21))
 (segment (start 83.4 120.1) (end 104.9201 120.1) (width 0.5) (layer "F.Cu") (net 21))
 (segment (start 131.2 91.557999) (end 131.2 89.8) (width 0.5) (layer "F.Cu") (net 21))
 (segment (start 134.64 86.36) (end 136.398 86.36) (width 0.5) (layer "F.Cu") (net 21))
 (segment (start 80.5 126.5) (end 80.5 123) (width 0.5) (layer "F.Cu") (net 21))
 (segment (start 104.9201 120.1) (end 117.2 107.820099) (width 0.5) (layer "F.Cu") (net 21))
 (segment (start 130.5 91.26805) (end 130.5 87.5) (width 0.5) (layer "F.Cu") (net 12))
 (segment (start 72.5 125) (end 78.1 119.4) (width 0.5) (layer "F.Cu") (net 12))
 (segment (start 116.5 105.26805) (end 130.5 91.26805) (width 0.5) (layer "F.Cu") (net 12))
 (segment (start 72.5 126.5) (end 72.5 125) (width 0.5) (layer "F.Cu") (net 12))
 (segment (start 130.5 87.5) (end 134.18 83.82) (width 0.5) (layer "F.Cu") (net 12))
 (segment (start 104.63015 119.4) (end 116.5 107.53015) (width 0.5) (layer "F.Cu") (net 12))
 (segment (start 116.5 107.53015) (end 116.5 105.26805) (width 0.5) (layer "F.Cu") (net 12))
 (segment (start 134.18 83.82) (end 136.398 83.82) (width 0.5) (layer "F.Cu") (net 12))
 (segment (start 78.1 119.4) (end 104.63015 119.4) (width 0.5) (layer "F.Cu") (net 12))
 (segment (start 115.8 104.9781) (end 129.8 90.9781) (width 0.5) (layer "F.Cu") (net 13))
 (segment (start 70.5 126.5) (end 70.5 124.5) (width 0.5) (layer "F.Cu") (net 13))
 (segment (start 115.8 107.2402) (end 115.8 104.9781) (width 0.5) (layer "F.Cu") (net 13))
 (segment (start 129.8 84.7) (end 133.22 81.28) (width 0.5) (layer "F.Cu") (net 13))
 (segment (start 129.8 90.9781) (end 129.8 84.7) (width 0.5) (layer "F.Cu") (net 13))
 (segment (start 133.22 81.28) (end 136.398 81.28) (width 0.5) (layer "F.Cu") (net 13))
 (segment (start 76.3 118.7) (end 104.3402 118.7) (width 0.5) (layer "F.Cu") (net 13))
 (segment (start 70.5 124.5) (end 76.3 118.7) (width 0.5) (layer "F.Cu") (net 13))
 (segment (start 104.3402 118.7) (end 115.8 107.2402) (width 0.5) (layer "F.Cu") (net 13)))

